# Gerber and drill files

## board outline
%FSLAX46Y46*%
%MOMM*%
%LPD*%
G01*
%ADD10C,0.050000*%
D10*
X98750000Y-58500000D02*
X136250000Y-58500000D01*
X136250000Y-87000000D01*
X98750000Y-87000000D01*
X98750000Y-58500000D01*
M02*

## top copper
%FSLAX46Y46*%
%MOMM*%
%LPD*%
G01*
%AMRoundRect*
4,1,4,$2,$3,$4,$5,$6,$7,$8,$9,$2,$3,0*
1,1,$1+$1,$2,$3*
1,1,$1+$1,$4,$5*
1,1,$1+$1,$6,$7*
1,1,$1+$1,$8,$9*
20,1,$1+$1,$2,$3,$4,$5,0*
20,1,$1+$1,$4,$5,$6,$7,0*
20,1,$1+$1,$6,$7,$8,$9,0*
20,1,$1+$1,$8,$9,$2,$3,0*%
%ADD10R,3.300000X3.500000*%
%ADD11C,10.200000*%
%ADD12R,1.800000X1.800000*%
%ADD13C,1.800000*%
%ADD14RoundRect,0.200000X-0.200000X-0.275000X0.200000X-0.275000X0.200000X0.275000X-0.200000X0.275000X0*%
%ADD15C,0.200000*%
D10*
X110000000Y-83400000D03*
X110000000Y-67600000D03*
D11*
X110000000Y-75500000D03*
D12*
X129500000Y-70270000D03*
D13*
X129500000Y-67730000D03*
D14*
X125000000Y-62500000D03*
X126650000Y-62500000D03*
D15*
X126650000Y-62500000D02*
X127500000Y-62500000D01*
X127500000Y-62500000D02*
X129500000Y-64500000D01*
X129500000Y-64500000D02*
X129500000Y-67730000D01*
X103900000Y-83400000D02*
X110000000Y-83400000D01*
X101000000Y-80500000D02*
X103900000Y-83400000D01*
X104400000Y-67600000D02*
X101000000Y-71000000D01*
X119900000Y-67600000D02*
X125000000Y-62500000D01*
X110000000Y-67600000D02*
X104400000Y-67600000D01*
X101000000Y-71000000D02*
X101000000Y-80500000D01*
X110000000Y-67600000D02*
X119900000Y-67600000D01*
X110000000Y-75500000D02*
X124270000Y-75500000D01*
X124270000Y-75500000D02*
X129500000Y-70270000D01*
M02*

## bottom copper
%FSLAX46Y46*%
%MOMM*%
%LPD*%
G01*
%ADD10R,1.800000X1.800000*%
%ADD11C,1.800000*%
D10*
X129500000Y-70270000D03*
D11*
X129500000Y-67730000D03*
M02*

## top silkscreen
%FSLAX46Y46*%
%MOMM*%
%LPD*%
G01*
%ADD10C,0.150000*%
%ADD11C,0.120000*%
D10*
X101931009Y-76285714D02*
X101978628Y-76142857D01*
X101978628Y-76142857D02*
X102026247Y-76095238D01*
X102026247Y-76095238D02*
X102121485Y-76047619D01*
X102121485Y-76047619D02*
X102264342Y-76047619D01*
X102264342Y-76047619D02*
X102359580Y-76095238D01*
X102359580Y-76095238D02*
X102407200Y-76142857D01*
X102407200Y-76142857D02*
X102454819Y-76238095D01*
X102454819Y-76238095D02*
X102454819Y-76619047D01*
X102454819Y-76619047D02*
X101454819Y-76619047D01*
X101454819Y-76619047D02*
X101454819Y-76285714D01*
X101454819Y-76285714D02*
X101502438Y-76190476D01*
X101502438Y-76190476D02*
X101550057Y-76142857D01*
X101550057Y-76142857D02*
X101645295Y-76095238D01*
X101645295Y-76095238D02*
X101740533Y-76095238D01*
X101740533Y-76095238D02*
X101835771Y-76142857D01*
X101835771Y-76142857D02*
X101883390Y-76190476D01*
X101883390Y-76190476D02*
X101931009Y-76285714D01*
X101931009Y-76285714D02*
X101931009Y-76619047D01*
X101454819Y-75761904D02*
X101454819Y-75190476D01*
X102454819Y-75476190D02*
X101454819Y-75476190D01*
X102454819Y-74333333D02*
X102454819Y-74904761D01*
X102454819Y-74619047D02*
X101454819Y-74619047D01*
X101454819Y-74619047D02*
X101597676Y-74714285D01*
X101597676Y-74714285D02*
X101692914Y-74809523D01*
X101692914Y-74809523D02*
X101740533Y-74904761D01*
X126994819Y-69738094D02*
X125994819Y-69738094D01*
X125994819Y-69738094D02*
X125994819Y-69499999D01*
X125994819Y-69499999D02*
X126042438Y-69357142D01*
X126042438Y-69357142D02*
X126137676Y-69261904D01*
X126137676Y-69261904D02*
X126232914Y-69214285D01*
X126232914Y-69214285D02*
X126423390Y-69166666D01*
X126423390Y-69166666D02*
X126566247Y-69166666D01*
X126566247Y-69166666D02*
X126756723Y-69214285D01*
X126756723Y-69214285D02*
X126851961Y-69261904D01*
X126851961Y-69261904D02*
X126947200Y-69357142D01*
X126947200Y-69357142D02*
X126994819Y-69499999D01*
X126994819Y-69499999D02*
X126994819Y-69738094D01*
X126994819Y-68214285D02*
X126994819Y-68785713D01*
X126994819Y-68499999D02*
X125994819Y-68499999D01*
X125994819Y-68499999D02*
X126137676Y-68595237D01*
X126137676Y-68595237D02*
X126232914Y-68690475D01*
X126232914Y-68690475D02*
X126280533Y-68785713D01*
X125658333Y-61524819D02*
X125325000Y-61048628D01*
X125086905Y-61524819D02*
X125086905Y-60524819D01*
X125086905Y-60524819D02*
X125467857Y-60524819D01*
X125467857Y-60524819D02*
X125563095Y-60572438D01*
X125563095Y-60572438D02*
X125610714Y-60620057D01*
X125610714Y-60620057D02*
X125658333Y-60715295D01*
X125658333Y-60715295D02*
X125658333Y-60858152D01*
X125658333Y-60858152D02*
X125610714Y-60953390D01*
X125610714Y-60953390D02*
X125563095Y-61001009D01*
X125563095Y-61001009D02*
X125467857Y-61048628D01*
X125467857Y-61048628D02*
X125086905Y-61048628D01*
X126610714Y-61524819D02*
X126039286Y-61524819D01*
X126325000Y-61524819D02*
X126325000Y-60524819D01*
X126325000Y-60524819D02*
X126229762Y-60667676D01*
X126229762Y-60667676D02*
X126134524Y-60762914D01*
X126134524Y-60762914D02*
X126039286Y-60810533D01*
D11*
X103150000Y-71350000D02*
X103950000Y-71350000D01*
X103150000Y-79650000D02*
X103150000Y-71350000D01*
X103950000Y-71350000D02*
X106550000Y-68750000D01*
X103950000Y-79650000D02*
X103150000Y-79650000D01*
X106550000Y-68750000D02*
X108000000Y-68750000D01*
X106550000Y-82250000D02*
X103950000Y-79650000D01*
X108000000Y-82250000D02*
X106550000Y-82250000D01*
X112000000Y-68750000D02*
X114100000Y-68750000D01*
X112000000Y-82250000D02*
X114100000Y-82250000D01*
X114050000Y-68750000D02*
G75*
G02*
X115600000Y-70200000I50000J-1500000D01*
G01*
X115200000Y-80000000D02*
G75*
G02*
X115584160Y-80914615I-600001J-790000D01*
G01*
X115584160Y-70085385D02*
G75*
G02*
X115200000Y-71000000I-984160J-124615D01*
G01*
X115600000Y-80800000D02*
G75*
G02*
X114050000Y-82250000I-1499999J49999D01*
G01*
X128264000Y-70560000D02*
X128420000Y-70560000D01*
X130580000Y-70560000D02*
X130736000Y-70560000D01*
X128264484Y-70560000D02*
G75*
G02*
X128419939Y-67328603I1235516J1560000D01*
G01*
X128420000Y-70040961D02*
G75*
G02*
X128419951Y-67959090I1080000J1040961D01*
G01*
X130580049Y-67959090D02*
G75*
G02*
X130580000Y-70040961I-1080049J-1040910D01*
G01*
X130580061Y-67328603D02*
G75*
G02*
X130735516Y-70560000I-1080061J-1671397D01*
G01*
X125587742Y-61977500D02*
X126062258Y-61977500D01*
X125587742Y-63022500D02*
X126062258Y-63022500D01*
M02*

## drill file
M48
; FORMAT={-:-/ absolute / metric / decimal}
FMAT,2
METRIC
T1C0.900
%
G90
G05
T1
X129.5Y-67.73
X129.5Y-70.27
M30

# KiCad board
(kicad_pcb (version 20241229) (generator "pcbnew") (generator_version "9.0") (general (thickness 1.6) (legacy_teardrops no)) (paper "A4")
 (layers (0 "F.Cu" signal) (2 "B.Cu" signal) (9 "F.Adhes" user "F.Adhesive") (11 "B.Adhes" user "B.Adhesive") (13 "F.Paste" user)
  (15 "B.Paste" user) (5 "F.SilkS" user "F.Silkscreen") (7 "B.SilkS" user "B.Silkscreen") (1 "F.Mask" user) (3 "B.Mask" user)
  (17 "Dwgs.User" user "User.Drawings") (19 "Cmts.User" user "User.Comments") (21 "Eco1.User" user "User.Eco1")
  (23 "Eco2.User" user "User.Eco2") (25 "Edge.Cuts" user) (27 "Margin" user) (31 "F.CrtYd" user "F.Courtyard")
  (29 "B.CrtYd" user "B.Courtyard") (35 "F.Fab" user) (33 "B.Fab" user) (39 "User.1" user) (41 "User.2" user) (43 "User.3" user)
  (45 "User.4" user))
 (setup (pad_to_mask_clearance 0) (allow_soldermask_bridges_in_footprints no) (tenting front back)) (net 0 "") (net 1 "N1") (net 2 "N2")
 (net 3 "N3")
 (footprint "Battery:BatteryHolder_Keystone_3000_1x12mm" (layer "F.Cu") (at 110 75.5 90)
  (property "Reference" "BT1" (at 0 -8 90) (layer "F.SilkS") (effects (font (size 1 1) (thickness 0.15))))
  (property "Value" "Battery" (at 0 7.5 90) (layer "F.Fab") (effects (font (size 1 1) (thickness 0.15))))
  (fp_line (start 4.15 -6.85) (end 4.15 -6.05) (stroke (width 0.12) (type solid)) (layer "F.SilkS"))
  (fp_line (start -4.15 -6.85) (end 4.15 -6.85) (stroke (width 0.12) (type solid)) (layer "F.SilkS"))
  (fp_line (start 4.15 -6.05) (end 6.75 -3.45) (stroke (width 0.12) (type solid)) (layer "F.SilkS"))
  (fp_line (start -4.15 -6.05) (end -4.15 -6.85) (stroke (width 0.12) (type solid)) (layer "F.SilkS"))
  (fp_line (start 6.75 -3.45) (end 6.75 -2) (stroke (width 0.12) (type solid)) (layer "F.SilkS"))
  (fp_line (start -6.75 -3.45) (end -4.15 -6.05) (stroke (width 0.12) (type solid)) (layer "F.SilkS"))
  (fp_line (start -6.75 -2) (end -6.75 -3.45) (stroke (width 0.12) (type solid)) (layer "F.SilkS"))
  (fp_line (start 6.75 2) (end 6.75 4.1) (stroke (width 0.12) (type solid)) (layer "F.SilkS"))
  (fp_line (start -6.75 2) (end -6.75 4.1) (stroke (width 0.12) (type solid)) (layer "F.SilkS"))
  (fp_arc (start 6.75 4.05) (mid 6.346016 5.125305) (end 5.3 5.6) (stroke (width 0.12) (type solid)) (layer "F.SilkS"))
  (fp_arc (start -4.5 5.2) (mid -4.90584 5.514615) (end -5.414615 5.58416) (stroke (width 0.12) (type solid)) (layer "F.SilkS"))
  (fp_arc (start 5.414615 5.58416) (mid 4.90584 5.514615) (end 4.5 5.2) (stroke (width 0.12) (type solid)) (layer "F.SilkS"))
  (fp_arc (start -5.3 5.6) (mid -6.346016 5.125305) (end -6.75 4.05) (stroke (width 0.12) (type solid)) (layer "F.SilkS"))
  (pad "1" smd rect (at -7.9 0 90) (size 3.5 3.3) (layers "F.Cu" "F.Mask" "F.Paste") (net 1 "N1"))
  (pad "1" smd rect (at 7.9 0 90) (size 3.5 3.3) (layers "F.Cu" "F.Mask" "F.Paste") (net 1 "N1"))
  (pad "2" smd circle (at 0 0 90) (size 10.2 10.2) (layers "F.Cu" "F.Mask") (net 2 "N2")))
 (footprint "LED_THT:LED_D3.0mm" (layer "F.Cu") (at 129.5 70.27 90)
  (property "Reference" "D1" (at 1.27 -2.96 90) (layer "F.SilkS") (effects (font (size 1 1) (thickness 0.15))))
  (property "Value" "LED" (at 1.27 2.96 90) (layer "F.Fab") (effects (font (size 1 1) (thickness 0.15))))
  (fp_line (start -0.29 -1.236) (end -0.29 -1.08) (stroke (width 0.12) (type solid)) (layer "F.SilkS"))
  (fp_line (start -0.29 1.08) (end -0.29 1.236) (stroke (width 0.12) (type solid)) (layer "F.SilkS"))
  (fp_arc (start -0.29 -1.235516) (mid 1.365624 -1.987701) (end 2.941397 -1.080061) (stroke (width 0.12) (type solid)) (layer "F.SilkS"))
  (fp_arc (start 0.229039 -1.08) (mid 1.269964 -1.5) (end 2.31091 -1.080049) (stroke (width 0.12) (type solid)) (layer "F.SilkS"))
  (fp_arc (start 2.31091 1.080049) (mid 1.269964 1.5) (end 0.229039 1.08) (stroke (width 0.12) (type solid)) (layer "F.SilkS"))
  (fp_arc (start 2.941397 1.080061) (mid 1.365624 1.987701) (end -0.29 1.235516) (stroke (width 0.12) (type solid)) (layer "F.SilkS"))
  (pad "1" thru_hole rect (at 0 0 90) (size 1.8 1.8) (drill 0.9) (layers "*.Cu" "*.Mask") (remove_unused_layers no) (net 2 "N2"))
  (pad "2" thru_hole circle (at 2.54 0 90) (size 1.8 1.8) (drill 0.9) (layers "*.Cu" "*.Mask") (remove_unused_layers no) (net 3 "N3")))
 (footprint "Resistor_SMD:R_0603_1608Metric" (layer "F.Cu") (at 125.825 62.5)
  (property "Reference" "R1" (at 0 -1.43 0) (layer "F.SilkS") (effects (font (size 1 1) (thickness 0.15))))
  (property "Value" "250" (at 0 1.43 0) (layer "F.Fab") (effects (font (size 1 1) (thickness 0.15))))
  (fp_line (start -0.237258 -0.5225) (end 0.237258 -0.5225) (stroke (width 0.12) (type solid)) (layer "F.SilkS"))
  (fp_line (start -0.237258 0.5225) (end 0.237258 0.5225) (stroke (width 0.12) (type solid)) (layer "F.SilkS"))
  (pad "1" smd roundrect (at -0.825 0) (size 0.8 0.95) (layers "F.Cu" "F.Mask" "F.Paste") (roundrect_rratio 0.25) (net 1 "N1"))
  (pad "2" smd roundrect (at 0.825 0) (size 0.8 0.95) (layers "F.Cu" "F.Mask" "F.Paste") (roundrect_rratio 0.25) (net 3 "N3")))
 (gr_rect (start 98.75 58.5) (end 136.25 87) (stroke (width 0.05) (type default)) (fill no) (layer "Edge.Cuts"))
 (segment (start 126.65 62.5) (end 127.5 62.5) (width 0.2) (layer "F.Cu") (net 3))
 (segment (start 127.5 62.5) (end 129.5 64.5) (width 0.2) (layer "F.Cu") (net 3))
 (segment (start 129.5 64.5) (end 129.5 67.73) (width 0.2) (layer "F.Cu") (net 3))
 (segment (start 103.9 83.4) (end 110 83.4) (width 0.2) (layer "F.Cu") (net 1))
 (segment (start 101 80.5) (end 103.9 83.4) (width 0.2) (layer "F.Cu") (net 1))
 (segment (start 104.4 67.6) (end 101 71) (width 0.2) (layer "F.Cu") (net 1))
 (segment (start 119.9 67.6) (end 125 62.5) (width 0.2) (layer "F.Cu") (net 1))
 (segment (start 110 67.6) (end 104.4 67.6) (width 0.2) (layer "F.Cu") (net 1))
 (segment (start 101 71) (end 101 80.5) (width 0.2) (layer "F.Cu") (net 1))
 (segment (start 110 67.6) (end 119.9 67.6) (width 0.2) (layer "F.Cu") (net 1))
 (segment (start 110 75.5) (end 124.27 75.5) (width 0.2) (layer "F.Cu") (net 2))
 (segment (start 124.27 75.5) (end 129.5 70.27) (width 0.2) (layer "F.Cu") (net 2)))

